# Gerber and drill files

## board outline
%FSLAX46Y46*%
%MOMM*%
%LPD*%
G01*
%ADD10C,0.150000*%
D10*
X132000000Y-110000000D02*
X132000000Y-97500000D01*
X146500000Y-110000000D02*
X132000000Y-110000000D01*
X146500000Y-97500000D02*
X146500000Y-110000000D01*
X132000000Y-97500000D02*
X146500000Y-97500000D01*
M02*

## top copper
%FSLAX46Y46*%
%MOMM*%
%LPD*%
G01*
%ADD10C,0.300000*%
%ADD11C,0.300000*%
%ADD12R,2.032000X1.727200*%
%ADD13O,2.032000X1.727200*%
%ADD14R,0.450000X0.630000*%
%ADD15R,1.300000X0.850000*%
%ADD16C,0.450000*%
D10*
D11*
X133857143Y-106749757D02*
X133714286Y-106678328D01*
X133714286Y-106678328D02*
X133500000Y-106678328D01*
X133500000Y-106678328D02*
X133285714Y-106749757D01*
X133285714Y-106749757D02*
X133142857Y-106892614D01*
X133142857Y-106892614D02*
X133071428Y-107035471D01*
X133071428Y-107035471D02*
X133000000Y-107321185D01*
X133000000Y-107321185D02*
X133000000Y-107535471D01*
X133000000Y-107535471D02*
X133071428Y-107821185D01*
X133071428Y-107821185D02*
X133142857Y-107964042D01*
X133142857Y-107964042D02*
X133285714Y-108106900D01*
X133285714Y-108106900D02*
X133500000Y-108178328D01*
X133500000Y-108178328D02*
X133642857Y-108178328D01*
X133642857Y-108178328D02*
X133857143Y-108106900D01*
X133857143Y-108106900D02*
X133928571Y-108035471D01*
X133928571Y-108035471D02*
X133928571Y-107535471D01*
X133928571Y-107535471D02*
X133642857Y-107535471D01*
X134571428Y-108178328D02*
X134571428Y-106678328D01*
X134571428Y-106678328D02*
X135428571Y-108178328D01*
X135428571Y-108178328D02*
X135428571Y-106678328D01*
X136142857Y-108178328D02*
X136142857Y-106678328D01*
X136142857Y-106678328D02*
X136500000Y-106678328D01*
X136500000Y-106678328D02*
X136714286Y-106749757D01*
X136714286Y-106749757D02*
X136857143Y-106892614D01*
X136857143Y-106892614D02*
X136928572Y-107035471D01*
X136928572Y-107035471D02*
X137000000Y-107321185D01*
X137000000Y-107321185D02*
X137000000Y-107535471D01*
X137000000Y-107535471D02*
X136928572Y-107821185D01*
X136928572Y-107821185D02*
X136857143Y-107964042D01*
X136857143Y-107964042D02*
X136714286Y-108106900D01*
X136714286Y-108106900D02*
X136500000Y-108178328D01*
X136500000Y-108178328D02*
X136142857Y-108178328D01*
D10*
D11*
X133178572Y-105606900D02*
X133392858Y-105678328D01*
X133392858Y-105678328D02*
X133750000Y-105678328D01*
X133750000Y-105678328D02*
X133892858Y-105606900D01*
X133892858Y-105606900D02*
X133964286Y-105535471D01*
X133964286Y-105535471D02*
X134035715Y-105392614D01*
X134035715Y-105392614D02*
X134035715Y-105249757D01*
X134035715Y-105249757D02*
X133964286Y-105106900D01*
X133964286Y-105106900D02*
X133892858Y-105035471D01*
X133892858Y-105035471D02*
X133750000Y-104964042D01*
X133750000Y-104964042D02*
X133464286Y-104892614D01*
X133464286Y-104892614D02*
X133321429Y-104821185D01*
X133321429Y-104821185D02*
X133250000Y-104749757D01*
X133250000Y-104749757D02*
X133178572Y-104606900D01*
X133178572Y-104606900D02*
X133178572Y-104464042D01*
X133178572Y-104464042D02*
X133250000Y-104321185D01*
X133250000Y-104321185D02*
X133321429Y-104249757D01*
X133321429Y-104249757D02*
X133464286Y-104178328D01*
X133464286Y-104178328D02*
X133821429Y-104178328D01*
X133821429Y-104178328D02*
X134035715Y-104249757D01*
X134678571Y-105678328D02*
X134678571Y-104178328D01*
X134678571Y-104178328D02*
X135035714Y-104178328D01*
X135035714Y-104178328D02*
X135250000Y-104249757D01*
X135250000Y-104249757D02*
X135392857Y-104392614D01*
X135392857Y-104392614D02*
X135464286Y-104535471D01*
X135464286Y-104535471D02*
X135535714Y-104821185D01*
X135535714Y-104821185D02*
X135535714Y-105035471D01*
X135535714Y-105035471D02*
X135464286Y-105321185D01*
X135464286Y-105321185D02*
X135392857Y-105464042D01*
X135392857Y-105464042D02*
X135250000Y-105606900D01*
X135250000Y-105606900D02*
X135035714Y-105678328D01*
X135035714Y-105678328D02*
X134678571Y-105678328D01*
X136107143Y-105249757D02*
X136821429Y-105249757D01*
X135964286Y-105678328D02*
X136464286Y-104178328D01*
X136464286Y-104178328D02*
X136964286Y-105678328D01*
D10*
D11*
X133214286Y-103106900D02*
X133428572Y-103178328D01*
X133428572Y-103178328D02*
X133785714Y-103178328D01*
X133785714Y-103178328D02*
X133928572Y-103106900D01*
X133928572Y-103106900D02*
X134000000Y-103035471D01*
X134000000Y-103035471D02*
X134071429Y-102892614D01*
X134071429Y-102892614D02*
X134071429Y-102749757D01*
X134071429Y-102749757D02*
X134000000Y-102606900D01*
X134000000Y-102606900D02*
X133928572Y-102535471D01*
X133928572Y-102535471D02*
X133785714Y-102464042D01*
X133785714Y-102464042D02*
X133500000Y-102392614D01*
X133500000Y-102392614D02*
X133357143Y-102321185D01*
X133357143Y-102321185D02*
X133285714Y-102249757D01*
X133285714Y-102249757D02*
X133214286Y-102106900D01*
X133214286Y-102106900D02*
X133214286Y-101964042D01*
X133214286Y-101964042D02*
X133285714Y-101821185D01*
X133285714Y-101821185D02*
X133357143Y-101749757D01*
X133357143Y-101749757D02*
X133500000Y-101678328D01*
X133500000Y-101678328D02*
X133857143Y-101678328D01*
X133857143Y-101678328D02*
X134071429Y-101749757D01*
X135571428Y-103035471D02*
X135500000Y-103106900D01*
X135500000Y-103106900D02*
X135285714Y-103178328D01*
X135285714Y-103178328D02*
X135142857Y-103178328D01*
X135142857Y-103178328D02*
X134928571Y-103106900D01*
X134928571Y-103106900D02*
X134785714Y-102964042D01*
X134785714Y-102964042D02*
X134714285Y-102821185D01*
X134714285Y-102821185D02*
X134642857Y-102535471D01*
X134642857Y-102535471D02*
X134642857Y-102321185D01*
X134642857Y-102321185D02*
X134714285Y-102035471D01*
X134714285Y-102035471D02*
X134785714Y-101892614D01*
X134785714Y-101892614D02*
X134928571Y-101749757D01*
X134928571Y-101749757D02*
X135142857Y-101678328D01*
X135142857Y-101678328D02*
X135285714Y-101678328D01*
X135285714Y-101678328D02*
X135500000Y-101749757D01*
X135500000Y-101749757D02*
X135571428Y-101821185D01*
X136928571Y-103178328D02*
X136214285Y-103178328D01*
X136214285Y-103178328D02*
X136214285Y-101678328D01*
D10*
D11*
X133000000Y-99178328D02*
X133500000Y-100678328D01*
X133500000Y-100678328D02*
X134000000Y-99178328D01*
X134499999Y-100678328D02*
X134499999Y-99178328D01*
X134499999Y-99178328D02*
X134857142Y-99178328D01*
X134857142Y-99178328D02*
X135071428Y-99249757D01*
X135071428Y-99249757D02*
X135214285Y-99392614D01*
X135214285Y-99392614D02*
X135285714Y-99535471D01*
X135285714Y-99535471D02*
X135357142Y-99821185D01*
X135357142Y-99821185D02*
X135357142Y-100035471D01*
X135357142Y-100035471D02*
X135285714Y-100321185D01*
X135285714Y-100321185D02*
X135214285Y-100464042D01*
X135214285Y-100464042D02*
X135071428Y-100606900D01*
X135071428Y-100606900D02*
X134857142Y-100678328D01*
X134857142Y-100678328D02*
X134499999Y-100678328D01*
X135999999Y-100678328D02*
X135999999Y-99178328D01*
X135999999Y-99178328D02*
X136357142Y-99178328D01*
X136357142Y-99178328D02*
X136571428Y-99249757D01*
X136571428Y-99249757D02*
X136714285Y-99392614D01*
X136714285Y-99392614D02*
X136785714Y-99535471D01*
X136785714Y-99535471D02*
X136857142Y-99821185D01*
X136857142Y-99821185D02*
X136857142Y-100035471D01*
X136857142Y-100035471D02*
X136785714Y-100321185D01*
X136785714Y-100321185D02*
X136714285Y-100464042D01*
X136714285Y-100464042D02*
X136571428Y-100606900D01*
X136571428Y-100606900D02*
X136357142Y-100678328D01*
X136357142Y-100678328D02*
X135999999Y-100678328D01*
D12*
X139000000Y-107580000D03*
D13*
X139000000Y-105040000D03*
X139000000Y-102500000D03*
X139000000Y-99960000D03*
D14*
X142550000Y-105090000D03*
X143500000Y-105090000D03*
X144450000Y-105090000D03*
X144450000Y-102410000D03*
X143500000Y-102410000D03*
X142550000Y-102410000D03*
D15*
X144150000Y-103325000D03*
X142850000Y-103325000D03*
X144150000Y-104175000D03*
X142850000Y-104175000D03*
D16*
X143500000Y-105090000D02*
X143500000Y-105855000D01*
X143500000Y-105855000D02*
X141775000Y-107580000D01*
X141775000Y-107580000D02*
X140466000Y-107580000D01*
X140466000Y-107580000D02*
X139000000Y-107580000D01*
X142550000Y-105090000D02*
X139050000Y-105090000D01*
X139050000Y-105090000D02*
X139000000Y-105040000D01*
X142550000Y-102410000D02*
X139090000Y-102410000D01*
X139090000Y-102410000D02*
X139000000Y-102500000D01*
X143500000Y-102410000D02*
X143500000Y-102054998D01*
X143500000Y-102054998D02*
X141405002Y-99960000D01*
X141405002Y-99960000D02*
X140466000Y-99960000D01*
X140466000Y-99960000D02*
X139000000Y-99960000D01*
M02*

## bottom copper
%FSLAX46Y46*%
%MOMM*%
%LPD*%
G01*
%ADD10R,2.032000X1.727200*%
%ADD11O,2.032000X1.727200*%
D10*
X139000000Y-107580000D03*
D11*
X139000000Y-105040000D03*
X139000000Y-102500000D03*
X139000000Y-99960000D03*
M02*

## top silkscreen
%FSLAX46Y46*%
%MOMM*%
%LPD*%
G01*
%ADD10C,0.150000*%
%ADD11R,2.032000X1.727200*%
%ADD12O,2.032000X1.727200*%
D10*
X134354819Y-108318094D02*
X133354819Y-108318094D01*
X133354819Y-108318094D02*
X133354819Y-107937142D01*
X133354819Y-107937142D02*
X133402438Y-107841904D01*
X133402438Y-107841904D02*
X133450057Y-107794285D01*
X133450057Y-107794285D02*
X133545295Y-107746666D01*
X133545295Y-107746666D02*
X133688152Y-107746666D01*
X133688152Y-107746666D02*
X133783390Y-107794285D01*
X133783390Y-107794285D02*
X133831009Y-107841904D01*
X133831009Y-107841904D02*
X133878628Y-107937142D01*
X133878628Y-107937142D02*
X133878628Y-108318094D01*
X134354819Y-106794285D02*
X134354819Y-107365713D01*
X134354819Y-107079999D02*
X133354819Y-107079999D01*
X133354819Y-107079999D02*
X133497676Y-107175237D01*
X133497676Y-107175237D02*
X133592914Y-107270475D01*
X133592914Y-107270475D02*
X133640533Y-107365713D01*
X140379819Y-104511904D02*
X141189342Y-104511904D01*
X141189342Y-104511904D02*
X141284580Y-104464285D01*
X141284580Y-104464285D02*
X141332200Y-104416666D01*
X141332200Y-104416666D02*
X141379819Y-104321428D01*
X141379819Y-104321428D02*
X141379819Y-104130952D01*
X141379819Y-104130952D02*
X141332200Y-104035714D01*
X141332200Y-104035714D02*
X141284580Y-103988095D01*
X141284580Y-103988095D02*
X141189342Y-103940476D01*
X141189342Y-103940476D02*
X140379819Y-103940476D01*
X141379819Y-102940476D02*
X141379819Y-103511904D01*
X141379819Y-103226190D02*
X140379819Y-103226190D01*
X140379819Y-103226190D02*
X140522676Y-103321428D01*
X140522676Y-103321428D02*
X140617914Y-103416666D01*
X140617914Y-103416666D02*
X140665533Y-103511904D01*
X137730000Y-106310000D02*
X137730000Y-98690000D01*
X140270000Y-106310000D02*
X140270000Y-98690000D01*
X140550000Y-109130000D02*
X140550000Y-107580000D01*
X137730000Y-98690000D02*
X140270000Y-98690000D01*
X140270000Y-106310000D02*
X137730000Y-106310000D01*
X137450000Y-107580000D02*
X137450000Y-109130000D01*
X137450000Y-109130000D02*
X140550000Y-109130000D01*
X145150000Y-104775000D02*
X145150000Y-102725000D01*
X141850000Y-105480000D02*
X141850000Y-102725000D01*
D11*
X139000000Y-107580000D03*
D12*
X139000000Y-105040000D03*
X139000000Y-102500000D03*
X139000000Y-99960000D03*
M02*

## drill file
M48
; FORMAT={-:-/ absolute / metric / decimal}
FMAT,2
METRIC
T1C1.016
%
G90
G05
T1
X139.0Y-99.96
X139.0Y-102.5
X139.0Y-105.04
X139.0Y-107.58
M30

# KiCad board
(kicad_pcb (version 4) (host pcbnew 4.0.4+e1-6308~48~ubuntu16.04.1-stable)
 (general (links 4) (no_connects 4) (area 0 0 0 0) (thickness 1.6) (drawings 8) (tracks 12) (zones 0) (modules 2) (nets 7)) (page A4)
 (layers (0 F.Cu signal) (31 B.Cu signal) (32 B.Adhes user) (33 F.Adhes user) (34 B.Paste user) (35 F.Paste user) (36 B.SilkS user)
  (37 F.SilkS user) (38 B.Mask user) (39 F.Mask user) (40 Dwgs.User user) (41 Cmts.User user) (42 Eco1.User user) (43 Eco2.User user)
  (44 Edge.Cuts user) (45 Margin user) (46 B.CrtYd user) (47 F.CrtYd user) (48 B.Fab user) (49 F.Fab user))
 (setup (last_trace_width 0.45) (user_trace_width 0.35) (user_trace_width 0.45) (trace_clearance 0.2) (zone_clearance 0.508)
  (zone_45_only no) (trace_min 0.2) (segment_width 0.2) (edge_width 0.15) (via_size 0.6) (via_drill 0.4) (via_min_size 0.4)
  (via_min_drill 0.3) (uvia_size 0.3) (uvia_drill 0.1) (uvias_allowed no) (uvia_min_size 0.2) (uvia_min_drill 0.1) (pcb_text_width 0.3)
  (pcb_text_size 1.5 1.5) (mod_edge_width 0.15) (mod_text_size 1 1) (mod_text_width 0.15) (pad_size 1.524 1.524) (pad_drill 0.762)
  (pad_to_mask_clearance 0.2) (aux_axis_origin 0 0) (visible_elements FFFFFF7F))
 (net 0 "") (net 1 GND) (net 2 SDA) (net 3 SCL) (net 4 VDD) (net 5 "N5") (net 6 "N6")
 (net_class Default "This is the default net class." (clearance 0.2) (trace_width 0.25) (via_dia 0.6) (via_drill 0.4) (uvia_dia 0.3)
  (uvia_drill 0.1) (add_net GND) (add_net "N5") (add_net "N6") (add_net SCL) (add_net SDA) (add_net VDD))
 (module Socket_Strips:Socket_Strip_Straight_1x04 (layer F.Cu) (at 139 107.58 90)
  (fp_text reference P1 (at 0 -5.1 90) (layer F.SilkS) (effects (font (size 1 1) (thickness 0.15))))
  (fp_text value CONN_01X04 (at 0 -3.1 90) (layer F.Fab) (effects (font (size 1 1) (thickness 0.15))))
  (fp_line (start 1.27 -1.27) (end 8.89 -1.27) (layer F.SilkS) (width 0.15))
  (fp_line (start 1.27 1.27) (end 8.89 1.27) (layer F.SilkS) (width 0.15))
  (fp_line (start -1.55 1.55) (end 0 1.55) (layer F.SilkS) (width 0.15))
  (fp_line (start 8.89 -1.27) (end 8.89 1.27) (layer F.SilkS) (width 0.15))
  (fp_line (start 1.27 1.27) (end 1.27 -1.27) (layer F.SilkS) (width 0.15))
  (fp_line (start 0 -1.55) (end -1.55 -1.55) (layer F.SilkS) (width 0.15))
  (fp_line (start -1.55 -1.55) (end -1.55 1.55) (layer F.SilkS) (width 0.15))
  (pad 1 thru_hole rect (at 0 0 90) (size 1.7272 2.032) (drill 1.016) (layers *.Cu *.Mask F.SilkS) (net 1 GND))
  (pad 2 thru_hole oval (at 2.54 0 90) (size 1.7272 2.032) (drill 1.016) (layers *.Cu *.Mask F.SilkS) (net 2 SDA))
  (pad 3 thru_hole oval (at 5.08 0 90) (size 1.7272 2.032) (drill 1.016) (layers *.Cu *.Mask F.SilkS) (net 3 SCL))
  (pad 4 thru_hole oval (at 7.62 0 90) (size 1.7272 2.032) (drill 1.016) (layers *.Cu *.Mask F.SilkS) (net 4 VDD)))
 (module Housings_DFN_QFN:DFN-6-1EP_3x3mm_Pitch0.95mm (layer F.Cu) (at 143.5 103.75 90)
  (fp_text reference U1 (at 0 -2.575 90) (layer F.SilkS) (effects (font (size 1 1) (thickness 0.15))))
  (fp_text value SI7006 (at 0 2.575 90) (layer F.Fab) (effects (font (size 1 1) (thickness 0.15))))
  (fp_line (start -1.025 1.65) (end 1.025 1.65) (layer F.SilkS) (width 0.15))
  (fp_line (start -1.73 -1.65) (end 1.025 -1.65) (layer F.SilkS) (width 0.15))
  (pad 1 smd rect (at -1.34 -0.95 90) (size 0.63 0.45) (layers F.Cu F.Paste F.Mask) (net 2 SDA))
  (pad 2 smd rect (at -1.34 0 90) (size 0.63 0.45) (layers F.Cu F.Paste F.Mask) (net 1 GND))
  (pad 3 smd rect (at -1.34 0.95 90) (size 0.63 0.45) (layers F.Cu F.Paste F.Mask) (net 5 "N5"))
  (pad 4 smd rect (at 1.34 0.95 90) (size 0.63 0.45) (layers F.Cu F.Paste F.Mask) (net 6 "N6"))
  (pad 5 smd rect (at 1.34 0 90) (size 0.63 0.45) (layers F.Cu F.Paste F.Mask) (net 4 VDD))
  (pad 6 smd rect (at 1.34 -0.95 90) (size 0.63 0.45) (layers F.Cu F.Paste F.Mask) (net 3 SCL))
  (pad 7 smd rect (at 0.425 0.65 90) (size 0.85 1.3) (layers F.Cu F.Paste F.Mask) (solder_paste_margin_ratio -0.2))
  (pad 7 smd rect (at 0.425 -0.65 90) (size 0.85 1.3) (layers F.Cu F.Paste F.Mask) (solder_paste_margin_ratio -0.2))
  (pad 7 smd rect (at -0.425 0.65 90) (size 0.85 1.3) (layers F.Cu F.Paste F.Mask) (solder_paste_margin_ratio -0.2))
  (pad 7 smd rect (at -0.425 -0.65 90) (size 0.85 1.3) (layers F.Cu F.Paste F.Mask) (solder_paste_margin_ratio -0.2)))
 (gr_line (start 132 110) (end 132 97.5) (layer Edge.Cuts) (width 0.15))
 (gr_line (start 146.5 110) (end 132 110) (layer Edge.Cuts) (width 0.15))
 (gr_line (start 146.5 97.5) (end 146.5 110) (layer Edge.Cuts) (width 0.15))
 (gr_line (start 132 97.5) (end 146.5 97.5) (layer Edge.Cuts) (width 0.15))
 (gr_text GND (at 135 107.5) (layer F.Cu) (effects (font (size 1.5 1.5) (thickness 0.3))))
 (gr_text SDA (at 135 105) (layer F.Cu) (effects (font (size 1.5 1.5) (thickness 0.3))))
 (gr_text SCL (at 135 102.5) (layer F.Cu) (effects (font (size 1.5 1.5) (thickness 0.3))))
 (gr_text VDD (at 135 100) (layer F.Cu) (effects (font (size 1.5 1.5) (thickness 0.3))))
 (segment (start 143.5 105.09) (end 143.5 105.855) (width 0.45) (layer F.Cu) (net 1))
 (segment (start 143.5 105.855) (end 141.775 107.58) (width 0.45) (layer F.Cu) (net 1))
 (segment (start 141.775 107.58) (end 140.466 107.58) (width 0.45) (layer F.Cu) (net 1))
 (segment (start 140.466 107.58) (end 139 107.58) (width 0.45) (layer F.Cu) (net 1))
 (segment (start 142.55 105.09) (end 139.05 105.09) (width 0.45) (layer F.Cu) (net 2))
 (segment (start 139.05 105.09) (end 139 105.04) (width 0.45) (layer F.Cu) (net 2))
 (segment (start 142.55 102.41) (end 139.09 102.41) (width 0.45) (layer F.Cu) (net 3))
 (segment (start 139.09 102.41) (end 139 102.5) (width 0.45) (layer F.Cu) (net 3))
 (segment (start 143.5 102.41) (end 143.5 102.054998) (width 0.45) (layer F.Cu) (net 4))
 (segment (start 143.5 102.054998) (end 141.405002 99.96) (width 0.45) (layer F.Cu) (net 4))
 (segment (start 141.405002 99.96) (end 140.466 99.96) (width 0.45) (layer F.Cu) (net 4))
 (segment (start 140.466 99.96) (end 139 99.96) (width 0.45) (layer F.Cu) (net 4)))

